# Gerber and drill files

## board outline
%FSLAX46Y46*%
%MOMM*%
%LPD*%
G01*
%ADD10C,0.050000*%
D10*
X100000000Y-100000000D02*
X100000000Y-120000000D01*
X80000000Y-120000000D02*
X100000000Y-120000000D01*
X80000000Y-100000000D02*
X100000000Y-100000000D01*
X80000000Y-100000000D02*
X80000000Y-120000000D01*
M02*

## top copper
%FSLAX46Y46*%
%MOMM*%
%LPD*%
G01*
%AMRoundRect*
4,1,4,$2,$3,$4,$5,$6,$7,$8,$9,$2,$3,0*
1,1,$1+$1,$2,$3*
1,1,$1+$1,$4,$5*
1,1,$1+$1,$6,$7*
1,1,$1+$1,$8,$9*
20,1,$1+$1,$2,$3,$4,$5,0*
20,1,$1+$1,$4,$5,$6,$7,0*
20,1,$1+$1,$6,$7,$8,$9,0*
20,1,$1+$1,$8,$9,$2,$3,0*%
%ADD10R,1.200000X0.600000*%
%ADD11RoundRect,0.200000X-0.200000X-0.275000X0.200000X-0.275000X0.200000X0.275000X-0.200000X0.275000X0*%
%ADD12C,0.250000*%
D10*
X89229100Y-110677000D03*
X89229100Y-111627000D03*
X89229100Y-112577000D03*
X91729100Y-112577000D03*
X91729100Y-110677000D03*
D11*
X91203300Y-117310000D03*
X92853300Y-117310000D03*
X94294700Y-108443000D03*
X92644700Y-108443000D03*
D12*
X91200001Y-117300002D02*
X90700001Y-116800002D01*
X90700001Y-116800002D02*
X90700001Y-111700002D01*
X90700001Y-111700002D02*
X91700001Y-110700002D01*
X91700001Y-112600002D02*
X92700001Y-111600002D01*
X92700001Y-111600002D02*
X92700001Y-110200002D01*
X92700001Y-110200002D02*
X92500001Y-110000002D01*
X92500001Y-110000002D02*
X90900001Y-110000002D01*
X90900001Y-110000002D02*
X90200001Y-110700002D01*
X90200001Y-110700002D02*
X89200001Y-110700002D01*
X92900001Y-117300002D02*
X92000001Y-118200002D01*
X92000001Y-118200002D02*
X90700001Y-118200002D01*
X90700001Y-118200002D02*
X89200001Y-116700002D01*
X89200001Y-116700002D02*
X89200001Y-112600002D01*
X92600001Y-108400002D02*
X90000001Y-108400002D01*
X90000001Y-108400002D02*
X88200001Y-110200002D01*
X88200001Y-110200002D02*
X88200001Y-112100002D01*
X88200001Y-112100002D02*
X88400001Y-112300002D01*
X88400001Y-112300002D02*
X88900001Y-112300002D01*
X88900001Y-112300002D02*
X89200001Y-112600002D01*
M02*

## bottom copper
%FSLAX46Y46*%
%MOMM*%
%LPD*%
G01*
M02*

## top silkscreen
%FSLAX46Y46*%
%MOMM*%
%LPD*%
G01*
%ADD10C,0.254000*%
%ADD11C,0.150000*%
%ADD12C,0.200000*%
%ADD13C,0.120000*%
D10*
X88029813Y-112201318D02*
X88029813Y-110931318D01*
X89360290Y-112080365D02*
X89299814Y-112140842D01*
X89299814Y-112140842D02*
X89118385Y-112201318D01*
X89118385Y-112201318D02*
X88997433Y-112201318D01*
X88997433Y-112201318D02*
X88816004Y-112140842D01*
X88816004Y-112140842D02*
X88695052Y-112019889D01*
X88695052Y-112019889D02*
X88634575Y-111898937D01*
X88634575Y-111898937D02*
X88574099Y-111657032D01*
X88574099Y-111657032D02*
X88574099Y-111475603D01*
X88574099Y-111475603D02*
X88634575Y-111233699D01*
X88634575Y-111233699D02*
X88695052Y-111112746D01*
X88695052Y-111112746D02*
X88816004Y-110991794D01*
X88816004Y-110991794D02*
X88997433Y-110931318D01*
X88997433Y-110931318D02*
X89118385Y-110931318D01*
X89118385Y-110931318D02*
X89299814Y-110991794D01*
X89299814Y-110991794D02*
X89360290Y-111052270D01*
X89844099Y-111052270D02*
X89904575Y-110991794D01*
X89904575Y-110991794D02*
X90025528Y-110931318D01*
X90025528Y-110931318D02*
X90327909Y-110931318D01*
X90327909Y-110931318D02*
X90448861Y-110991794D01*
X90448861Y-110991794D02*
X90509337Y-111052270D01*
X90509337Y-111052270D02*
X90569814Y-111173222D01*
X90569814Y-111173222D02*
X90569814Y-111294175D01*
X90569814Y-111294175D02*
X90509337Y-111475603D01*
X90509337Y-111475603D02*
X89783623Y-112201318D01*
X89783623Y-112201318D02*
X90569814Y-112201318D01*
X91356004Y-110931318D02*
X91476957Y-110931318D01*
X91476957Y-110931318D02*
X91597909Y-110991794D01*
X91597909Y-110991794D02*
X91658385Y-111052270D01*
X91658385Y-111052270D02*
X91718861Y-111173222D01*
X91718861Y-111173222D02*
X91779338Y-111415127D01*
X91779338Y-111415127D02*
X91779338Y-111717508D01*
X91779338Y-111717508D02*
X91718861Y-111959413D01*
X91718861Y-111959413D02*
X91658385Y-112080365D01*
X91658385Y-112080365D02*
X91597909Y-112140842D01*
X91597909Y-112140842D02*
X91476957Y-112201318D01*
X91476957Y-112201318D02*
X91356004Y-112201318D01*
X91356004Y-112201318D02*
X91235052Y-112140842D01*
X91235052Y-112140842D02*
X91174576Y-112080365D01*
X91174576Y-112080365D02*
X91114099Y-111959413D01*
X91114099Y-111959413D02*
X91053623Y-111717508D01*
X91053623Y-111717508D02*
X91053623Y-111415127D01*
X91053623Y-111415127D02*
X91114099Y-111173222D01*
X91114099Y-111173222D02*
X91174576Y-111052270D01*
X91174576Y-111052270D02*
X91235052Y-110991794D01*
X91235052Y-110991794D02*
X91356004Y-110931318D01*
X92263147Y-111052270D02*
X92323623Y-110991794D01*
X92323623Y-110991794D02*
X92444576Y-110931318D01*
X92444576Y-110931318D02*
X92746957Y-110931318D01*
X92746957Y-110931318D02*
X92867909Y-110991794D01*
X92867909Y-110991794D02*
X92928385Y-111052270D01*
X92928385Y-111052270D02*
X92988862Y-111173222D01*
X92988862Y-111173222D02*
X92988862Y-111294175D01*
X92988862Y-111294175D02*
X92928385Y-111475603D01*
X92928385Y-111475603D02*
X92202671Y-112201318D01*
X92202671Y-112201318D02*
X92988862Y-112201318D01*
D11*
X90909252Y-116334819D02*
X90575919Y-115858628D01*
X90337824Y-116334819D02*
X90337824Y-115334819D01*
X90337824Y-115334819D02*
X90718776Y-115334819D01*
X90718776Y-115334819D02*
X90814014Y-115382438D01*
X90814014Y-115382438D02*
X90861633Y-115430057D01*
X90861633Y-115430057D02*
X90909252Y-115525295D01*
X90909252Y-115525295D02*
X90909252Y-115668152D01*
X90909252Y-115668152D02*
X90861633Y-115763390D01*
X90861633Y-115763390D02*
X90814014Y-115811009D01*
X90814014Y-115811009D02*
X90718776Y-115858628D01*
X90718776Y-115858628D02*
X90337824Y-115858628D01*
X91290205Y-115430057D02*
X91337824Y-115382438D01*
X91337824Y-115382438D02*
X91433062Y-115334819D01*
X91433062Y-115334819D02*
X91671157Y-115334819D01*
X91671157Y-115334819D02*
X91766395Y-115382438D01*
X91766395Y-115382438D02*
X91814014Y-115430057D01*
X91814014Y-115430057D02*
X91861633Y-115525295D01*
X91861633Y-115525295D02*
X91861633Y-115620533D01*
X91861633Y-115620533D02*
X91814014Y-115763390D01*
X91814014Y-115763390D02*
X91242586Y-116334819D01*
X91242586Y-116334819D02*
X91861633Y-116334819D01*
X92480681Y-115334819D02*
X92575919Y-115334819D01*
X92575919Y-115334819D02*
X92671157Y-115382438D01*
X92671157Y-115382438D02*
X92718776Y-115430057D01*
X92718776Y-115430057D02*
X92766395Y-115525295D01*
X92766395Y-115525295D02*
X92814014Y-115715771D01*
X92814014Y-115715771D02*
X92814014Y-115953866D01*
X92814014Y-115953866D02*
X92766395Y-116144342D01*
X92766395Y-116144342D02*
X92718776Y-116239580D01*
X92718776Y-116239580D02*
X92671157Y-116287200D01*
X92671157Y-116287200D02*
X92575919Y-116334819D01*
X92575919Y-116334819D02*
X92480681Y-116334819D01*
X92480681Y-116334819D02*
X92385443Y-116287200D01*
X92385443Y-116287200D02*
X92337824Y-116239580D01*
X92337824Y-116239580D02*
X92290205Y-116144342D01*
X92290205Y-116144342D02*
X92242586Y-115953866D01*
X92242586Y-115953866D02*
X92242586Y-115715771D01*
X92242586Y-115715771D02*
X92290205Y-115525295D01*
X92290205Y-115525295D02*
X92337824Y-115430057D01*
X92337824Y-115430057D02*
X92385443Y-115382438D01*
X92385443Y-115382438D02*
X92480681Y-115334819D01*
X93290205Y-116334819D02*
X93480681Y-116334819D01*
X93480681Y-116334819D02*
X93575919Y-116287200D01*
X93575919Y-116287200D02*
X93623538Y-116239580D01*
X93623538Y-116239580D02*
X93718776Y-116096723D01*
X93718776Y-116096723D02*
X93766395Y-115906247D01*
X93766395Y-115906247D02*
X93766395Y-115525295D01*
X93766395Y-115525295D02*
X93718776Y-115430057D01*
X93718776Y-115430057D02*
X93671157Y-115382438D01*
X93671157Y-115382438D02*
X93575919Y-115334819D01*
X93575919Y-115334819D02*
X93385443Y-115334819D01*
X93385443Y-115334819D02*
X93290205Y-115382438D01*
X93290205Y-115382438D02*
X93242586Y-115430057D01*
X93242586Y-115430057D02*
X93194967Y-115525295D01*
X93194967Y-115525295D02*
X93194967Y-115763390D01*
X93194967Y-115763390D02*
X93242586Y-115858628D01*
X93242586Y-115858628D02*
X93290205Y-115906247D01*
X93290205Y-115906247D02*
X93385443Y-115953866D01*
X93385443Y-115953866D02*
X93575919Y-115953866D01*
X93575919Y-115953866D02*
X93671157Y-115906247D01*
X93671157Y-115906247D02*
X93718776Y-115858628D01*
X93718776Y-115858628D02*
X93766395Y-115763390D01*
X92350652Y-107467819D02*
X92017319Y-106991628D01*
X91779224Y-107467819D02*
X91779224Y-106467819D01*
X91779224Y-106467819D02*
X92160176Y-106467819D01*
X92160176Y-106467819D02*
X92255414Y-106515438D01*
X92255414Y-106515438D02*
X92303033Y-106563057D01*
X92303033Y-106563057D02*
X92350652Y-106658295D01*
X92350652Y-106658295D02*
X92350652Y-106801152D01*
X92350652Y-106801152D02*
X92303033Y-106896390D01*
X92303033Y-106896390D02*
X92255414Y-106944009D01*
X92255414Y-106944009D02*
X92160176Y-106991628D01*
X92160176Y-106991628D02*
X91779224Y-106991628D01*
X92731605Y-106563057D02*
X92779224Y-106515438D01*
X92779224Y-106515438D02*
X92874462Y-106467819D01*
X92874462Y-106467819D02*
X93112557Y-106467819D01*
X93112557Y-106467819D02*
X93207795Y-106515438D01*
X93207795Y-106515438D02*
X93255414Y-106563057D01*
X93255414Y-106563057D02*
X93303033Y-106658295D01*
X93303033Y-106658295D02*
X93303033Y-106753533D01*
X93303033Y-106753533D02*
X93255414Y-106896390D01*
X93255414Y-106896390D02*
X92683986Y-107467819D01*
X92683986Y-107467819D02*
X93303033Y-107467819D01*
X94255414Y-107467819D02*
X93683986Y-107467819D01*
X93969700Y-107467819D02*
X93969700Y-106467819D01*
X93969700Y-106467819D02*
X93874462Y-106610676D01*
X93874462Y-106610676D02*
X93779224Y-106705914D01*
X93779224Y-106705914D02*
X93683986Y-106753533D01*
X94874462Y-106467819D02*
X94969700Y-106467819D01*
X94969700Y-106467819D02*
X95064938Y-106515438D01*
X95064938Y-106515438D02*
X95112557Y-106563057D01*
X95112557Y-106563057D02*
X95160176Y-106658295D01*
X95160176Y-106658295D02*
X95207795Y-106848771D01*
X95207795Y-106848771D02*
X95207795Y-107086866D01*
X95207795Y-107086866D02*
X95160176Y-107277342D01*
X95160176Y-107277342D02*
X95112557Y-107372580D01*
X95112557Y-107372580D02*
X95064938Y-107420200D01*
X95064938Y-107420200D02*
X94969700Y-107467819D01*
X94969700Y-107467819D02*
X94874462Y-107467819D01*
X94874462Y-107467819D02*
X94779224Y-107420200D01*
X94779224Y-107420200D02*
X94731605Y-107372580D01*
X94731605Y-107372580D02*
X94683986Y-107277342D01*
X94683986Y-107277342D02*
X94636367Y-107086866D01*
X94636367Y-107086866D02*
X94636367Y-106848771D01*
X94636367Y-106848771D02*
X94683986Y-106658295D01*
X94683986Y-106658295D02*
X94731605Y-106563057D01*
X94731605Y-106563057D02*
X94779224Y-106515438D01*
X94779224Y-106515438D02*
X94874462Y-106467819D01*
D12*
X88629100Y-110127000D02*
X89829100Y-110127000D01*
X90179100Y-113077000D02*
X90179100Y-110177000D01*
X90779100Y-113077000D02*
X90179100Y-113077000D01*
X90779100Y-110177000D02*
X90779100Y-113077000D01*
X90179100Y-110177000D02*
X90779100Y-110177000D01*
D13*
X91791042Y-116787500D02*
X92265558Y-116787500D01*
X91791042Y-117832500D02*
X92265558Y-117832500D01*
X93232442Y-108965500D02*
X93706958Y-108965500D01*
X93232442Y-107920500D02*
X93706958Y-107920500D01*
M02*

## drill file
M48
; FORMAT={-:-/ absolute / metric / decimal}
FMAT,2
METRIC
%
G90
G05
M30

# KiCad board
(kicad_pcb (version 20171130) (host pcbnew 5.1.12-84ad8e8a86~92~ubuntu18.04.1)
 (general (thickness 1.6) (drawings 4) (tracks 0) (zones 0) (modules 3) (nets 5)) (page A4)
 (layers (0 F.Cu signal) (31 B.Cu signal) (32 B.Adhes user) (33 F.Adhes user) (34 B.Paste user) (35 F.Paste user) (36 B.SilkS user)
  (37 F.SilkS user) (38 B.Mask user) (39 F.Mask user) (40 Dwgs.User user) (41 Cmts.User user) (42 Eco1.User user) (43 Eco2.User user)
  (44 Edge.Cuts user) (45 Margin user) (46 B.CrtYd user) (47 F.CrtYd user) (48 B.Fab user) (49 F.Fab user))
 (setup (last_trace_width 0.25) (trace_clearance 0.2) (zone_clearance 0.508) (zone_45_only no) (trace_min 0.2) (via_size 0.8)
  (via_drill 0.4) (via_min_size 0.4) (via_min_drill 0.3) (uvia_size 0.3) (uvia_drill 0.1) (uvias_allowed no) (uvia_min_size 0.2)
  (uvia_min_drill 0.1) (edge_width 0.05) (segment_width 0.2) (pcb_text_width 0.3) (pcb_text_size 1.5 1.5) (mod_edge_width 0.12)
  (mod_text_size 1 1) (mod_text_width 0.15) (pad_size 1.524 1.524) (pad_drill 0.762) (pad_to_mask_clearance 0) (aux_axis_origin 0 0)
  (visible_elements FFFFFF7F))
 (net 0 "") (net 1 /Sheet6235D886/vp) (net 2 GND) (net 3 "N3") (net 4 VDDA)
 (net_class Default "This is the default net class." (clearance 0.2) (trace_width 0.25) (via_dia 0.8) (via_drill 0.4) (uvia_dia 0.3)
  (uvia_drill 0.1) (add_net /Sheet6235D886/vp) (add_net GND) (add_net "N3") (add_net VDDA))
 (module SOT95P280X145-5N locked (layer F.Cu) (at 90.479100 111.627000)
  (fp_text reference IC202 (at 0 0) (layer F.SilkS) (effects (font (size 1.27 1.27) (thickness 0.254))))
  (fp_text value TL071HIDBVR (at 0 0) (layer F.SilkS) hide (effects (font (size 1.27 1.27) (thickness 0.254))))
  (fp_line (start -1.85 -1.5) (end -0.65 -1.5) (layer F.SilkS) (width 0.2))
  (fp_line (start -0.3 1.45) (end -0.3 -1.45) (layer F.SilkS) (width 0.2))
  (fp_line (start 0.3 1.45) (end -0.3 1.45) (layer F.SilkS) (width 0.2))
  (fp_line (start 0.3 -1.45) (end 0.3 1.45) (layer F.SilkS) (width 0.2))
  (fp_line (start -0.3 -1.45) (end 0.3 -1.45) (layer F.SilkS) (width 0.2))
  (pad 1 smd rect (at -1.25 -0.95 90.000000) (size 0.6 1.2) (layers F.Cu F.Mask F.Paste) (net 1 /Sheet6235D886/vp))
  (pad 2 smd rect (at -1.25 0 90.000000) (size 0.6 1.2) (layers F.Cu F.Mask F.Paste) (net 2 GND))
  (pad 3 smd rect (at -1.25 0.95 90.000000) (size 0.6 1.2) (layers F.Cu F.Mask F.Paste) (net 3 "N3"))
  (pad 4 smd rect (at 1.25 0.95 90.000000) (size 0.6 1.2) (layers F.Cu F.Mask F.Paste) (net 1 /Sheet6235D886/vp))
  (pad 5 smd rect (at 1.25 -0.95 90.000000) (size 0.6 1.2) (layers F.Cu F.Mask F.Paste) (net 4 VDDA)))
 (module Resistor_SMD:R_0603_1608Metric (layer F.Cu) (at 92.028300 117.310000)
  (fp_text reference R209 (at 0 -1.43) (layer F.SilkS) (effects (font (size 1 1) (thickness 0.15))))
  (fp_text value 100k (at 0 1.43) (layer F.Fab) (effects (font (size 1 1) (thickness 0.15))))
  (fp_line (start -0.237258 -0.5225) (end 0.237258 -0.5225) (layer F.SilkS) (width 0.12))
  (fp_line (start -0.237258 0.5225) (end 0.237258 0.5225) (layer F.SilkS) (width 0.12))
  (pad 1 smd roundrect (at -0.825 0) (size 0.8 0.95) (layers F.Cu F.Mask F.Paste) (roundrect_rratio 0.25) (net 4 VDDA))
  (pad 2 smd roundrect (at 0.825 0) (size 0.8 0.95) (layers F.Cu F.Mask F.Paste) (roundrect_rratio 0.25) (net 3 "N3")))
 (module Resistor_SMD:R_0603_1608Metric (layer F.Cu) (at 93.469700 108.443000)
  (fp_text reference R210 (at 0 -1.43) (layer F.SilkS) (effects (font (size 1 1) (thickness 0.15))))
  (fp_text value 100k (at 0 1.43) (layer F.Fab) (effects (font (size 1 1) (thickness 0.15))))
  (fp_line (start -0.237258 0.5225) (end 0.237258 0.5225) (layer F.SilkS) (width 0.12))
  (fp_line (start -0.237258 -0.5225) (end 0.237258 -0.5225) (layer F.SilkS) (width 0.12))
  (pad 2 smd roundrect (at 0.825 0) (size 0.8 0.95) (layers F.Cu F.Mask F.Paste) (roundrect_rratio 0.25) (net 2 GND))
  (pad 1 smd roundrect (at -0.825 0) (size 0.8 0.95) (layers F.Cu F.Mask F.Paste) (roundrect_rratio 0.25) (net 3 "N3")))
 (gr_line (start 100 100) (end 100 120) (layer Edge.Cuts) (width 0.05))
 (gr_line (start 80 120) (end 100 120) (layer Edge.Cuts) (width 0.05))
 (gr_line (start 80 100) (end 100 100) (layer Edge.Cuts) (width 0.05))
 (gr_line (start 80 100) (end 80 120) (layer Edge.Cuts) (width 0.05))
 (segment (start 91.200001 117.300002) (end 90.700001 116.800002) (width 0.250000) (layer F.Cu) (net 4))
 (segment (start 90.700001 116.800002) (end 90.700001 111.700002) (width 0.250000) (layer F.Cu) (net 4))
 (segment (start 90.700001 111.700002) (end 91.700001 110.700002) (width 0.250000) (layer F.Cu) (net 4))
 (segment (start 91.700001 112.600002) (end 92.700001 111.600002) (width 0.250000) (layer F.Cu) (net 1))
 (segment (start 92.700001 111.600002) (end 92.700001 110.200002) (width 0.250000) (layer F.Cu) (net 1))
 (segment (start 92.700001 110.200002) (end 92.500001 110.000002) (width 0.250000) (layer F.Cu) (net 1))
 (segment (start 92.500001 110.000002) (end 90.900001 110.000002) (width 0.250000) (layer F.Cu) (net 1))
 (segment (start 90.900001 110.000002) (end 90.200001 110.700002) (width 0.250000) (layer F.Cu) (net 1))
 (segment (start 90.200001 110.700002) (end 89.200001 110.700002) (width 0.250000) (layer F.Cu) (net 1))
 (segment (start 92.900001 117.300002) (end 92.000001 118.200002) (width 0.250000) (layer F.Cu) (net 3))
 (segment (start 92.000001 118.200002) (end 90.700001 118.200002) (width 0.250000) (layer F.Cu) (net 3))
 (segment (start 90.700001 118.200002) (end 89.200001 116.700002) (width 0.250000) (layer F.Cu) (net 3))
 (segment (start 89.200001 116.700002) (end 89.200001 112.600002) (width 0.250000) (layer F.Cu) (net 3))
 (segment (start 92.600001 108.400002) (end 90.000001 108.400002) (width 0.250000) (layer F.Cu) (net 3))
 (segment (start 90.000001 108.400002) (end 88.200001 110.200002) (width 0.250000) (layer F.Cu) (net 3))
 (segment (start 88.200001 110.200002) (end 88.200001 112.100002) (width 0.250000) (layer F.Cu) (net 3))
 (segment (start 88.200001 112.100002) (end 88.400001 112.300002) (width 0.250000) (layer F.Cu) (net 3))
 (segment (start 88.400001 112.300002) (end 88.900001 112.300002) (width 0.250000) (layer F.Cu) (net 3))
 (segment (start 88.900001 112.300002) (end 89.200001 112.600002) (width 0.250000) (layer F.Cu) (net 3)))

